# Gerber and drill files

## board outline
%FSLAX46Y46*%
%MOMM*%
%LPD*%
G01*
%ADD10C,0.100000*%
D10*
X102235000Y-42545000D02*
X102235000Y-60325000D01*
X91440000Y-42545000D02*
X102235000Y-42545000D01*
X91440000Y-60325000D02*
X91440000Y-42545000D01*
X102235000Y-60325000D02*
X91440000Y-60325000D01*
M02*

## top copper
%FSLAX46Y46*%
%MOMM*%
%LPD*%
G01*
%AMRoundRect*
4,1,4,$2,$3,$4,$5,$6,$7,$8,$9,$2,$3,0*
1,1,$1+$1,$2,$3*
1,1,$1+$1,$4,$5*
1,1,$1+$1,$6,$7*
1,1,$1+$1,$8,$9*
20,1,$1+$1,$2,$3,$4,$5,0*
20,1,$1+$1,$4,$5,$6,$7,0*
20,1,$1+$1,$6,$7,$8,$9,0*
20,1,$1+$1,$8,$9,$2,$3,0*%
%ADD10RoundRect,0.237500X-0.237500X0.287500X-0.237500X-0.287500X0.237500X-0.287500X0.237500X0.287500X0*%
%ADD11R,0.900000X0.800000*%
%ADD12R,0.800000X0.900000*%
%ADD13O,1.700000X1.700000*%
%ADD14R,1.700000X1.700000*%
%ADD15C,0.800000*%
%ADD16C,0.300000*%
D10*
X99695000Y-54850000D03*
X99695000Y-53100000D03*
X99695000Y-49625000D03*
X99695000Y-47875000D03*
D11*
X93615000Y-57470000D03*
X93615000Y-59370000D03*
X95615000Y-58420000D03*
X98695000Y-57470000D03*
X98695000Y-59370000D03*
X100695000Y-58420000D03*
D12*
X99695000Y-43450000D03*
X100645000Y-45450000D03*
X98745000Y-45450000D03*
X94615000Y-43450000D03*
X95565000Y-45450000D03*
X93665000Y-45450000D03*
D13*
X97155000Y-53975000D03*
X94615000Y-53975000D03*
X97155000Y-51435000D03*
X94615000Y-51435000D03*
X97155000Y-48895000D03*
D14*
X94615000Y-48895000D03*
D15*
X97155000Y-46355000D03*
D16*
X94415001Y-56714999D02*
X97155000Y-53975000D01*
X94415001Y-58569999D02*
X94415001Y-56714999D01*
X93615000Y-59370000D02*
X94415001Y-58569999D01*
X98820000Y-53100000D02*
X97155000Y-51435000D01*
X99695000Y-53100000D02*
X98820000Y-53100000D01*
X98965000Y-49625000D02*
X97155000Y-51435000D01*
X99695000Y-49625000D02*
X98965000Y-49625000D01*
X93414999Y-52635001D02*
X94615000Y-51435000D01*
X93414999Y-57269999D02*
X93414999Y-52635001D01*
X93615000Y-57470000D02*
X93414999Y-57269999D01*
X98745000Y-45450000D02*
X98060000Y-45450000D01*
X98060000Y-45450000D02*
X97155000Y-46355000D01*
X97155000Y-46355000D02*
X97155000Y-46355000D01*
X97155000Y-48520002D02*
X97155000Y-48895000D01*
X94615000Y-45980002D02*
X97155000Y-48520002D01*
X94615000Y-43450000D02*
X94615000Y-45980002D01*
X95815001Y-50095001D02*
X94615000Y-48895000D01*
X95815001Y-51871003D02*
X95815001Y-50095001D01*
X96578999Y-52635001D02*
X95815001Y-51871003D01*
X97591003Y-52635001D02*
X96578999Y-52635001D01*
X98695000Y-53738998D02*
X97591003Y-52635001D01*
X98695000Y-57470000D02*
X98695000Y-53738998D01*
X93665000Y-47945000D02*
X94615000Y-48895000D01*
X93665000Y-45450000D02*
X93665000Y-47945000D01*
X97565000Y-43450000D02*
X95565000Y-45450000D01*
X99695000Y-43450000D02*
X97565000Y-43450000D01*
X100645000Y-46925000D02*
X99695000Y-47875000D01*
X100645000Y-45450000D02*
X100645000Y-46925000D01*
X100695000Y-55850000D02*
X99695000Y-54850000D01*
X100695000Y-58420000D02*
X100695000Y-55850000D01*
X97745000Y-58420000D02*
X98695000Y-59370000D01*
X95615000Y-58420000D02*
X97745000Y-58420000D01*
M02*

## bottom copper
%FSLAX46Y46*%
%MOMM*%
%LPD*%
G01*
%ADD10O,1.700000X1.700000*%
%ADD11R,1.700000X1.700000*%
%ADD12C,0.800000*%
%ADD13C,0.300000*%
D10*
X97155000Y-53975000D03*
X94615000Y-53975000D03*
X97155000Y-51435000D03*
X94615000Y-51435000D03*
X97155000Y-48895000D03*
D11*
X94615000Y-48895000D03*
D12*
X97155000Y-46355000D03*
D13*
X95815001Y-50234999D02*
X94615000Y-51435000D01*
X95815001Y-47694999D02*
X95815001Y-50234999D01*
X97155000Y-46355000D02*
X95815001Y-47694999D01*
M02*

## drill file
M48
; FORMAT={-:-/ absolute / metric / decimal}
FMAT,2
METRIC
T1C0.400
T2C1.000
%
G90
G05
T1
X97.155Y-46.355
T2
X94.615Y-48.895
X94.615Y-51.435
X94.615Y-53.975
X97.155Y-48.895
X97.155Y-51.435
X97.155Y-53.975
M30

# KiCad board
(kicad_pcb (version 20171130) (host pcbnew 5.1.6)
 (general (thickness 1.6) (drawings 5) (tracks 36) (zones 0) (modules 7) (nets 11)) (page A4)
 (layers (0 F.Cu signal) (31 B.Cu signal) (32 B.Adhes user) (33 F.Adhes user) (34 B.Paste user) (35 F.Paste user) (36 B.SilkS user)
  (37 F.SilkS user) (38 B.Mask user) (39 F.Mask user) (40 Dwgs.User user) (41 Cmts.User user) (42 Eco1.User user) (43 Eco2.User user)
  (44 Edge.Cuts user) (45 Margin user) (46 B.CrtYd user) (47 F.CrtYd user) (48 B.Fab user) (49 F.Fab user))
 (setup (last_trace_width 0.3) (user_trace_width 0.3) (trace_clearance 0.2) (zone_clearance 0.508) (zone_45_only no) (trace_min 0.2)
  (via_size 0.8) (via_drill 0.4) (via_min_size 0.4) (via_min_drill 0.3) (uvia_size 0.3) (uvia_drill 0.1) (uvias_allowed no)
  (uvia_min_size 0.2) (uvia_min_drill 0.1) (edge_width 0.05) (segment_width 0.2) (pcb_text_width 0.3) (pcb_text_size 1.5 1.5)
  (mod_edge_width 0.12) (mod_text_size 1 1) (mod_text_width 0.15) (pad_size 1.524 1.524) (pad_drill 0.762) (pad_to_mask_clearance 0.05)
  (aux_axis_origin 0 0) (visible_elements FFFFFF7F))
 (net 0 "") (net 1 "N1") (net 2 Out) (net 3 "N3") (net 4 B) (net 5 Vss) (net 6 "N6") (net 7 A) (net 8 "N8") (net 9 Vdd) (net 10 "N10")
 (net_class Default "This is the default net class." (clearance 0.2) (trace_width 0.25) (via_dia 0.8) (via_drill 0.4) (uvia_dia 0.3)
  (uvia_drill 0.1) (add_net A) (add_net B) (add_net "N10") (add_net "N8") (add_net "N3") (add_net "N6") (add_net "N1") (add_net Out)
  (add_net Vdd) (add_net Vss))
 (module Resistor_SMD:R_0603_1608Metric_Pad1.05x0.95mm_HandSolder (layer F.Cu) (at 99.695 53.975 270)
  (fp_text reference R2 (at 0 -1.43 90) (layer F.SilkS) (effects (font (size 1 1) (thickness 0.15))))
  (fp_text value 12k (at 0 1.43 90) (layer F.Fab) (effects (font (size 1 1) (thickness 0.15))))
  (pad 2 smd roundrect (at 0.875 0 270) (size 1.05 0.95) (layers F.Cu F.Paste F.Mask) (roundrect_rratio 0.25) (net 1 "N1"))
  (pad 1 smd roundrect (at -0.875 0 270) (size 1.05 0.95) (layers F.Cu F.Paste F.Mask) (roundrect_rratio 0.25) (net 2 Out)))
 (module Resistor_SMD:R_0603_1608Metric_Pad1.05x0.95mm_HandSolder (layer F.Cu) (at 99.695 48.75 270)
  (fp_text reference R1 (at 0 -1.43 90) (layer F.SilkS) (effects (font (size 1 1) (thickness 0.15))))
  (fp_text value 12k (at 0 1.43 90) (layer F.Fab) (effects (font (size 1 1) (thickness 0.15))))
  (pad 2 smd roundrect (at 0.875 0 270) (size 1.05 0.95) (layers F.Cu F.Paste F.Mask) (roundrect_rratio 0.25) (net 2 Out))
  (pad 1 smd roundrect (at -0.875 0 270) (size 1.05 0.95) (layers F.Cu F.Paste F.Mask) (roundrect_rratio 0.25) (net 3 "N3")))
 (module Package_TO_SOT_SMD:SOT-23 (layer F.Cu) (at 94.615 58.42)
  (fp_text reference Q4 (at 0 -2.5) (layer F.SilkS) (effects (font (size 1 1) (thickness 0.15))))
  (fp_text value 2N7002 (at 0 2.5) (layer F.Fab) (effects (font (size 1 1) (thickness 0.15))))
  (pad 1 smd rect (at -1 -0.95) (size 0.9 0.8) (layers F.Cu F.Paste F.Mask) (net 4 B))
  (pad 2 smd rect (at -1 0.95) (size 0.9 0.8) (layers F.Cu F.Paste F.Mask) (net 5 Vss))
  (pad 3 smd rect (at 1 0) (size 0.9 0.8) (layers F.Cu F.Paste F.Mask) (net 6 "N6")))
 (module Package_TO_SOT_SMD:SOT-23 (layer F.Cu) (at 99.695 58.42)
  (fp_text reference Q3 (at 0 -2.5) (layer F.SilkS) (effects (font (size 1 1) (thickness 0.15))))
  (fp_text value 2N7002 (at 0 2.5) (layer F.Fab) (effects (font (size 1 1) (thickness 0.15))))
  (pad 1 smd rect (at -1 -0.95) (size 0.9 0.8) (layers F.Cu F.Paste F.Mask) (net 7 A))
  (pad 2 smd rect (at -1 0.95) (size 0.9 0.8) (layers F.Cu F.Paste F.Mask) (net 6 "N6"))
  (pad 3 smd rect (at 1 0) (size 0.9 0.8) (layers F.Cu F.Paste F.Mask) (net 1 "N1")))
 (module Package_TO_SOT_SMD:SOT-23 (layer F.Cu) (at 99.695 44.45 90)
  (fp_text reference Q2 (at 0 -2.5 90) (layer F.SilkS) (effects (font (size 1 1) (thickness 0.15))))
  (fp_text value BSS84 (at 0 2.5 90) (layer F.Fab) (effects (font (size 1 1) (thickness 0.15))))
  (pad 3 smd rect (at 1 0 90) (size 0.9 0.8) (layers F.Cu F.Paste F.Mask) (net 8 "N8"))
  (pad 2 smd rect (at -1 0.95 90) (size 0.9 0.8) (layers F.Cu F.Paste F.Mask) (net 3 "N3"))
  (pad 1 smd rect (at -1 -0.95 90) (size 0.9 0.8) (layers F.Cu F.Paste F.Mask) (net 4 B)))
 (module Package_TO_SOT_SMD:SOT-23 (layer F.Cu) (at 94.615 44.45 90)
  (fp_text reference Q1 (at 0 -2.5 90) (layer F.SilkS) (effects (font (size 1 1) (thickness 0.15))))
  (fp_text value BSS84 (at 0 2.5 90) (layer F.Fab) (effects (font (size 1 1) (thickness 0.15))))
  (pad 3 smd rect (at 1 0 90) (size 0.9 0.8) (layers F.Cu F.Paste F.Mask) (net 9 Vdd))
  (pad 2 smd rect (at -1 0.95 90) (size 0.9 0.8) (layers F.Cu F.Paste F.Mask) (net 8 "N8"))
  (pad 1 smd rect (at -1 -0.95 90) (size 0.9 0.8) (layers F.Cu F.Paste F.Mask) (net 7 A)))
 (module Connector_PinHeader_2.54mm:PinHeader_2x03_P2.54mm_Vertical (layer F.Cu) (at 94.615 48.895)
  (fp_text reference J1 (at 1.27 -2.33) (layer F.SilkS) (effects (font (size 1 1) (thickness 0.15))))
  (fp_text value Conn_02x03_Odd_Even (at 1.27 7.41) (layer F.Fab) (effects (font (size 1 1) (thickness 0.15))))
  (pad 6 thru_hole oval (at 2.54 5.08) (size 1.7 1.7) (drill 1) (layers *.Cu *.Mask) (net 5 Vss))
  (pad 5 thru_hole oval (at 0 5.08) (size 1.7 1.7) (drill 1) (layers *.Cu *.Mask) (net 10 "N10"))
  (pad 4 thru_hole oval (at 2.54 2.54) (size 1.7 1.7) (drill 1) (layers *.Cu *.Mask) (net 2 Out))
  (pad 3 thru_hole oval (at 0 2.54) (size 1.7 1.7) (drill 1) (layers *.Cu *.Mask) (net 4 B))
  (pad 2 thru_hole oval (at 2.54 0) (size 1.7 1.7) (drill 1) (layers *.Cu *.Mask) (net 9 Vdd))
  (pad 1 thru_hole rect (at 0 0) (size 1.7 1.7) (drill 1) (layers *.Cu *.Mask) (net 7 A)))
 (gr_line (start 102.235 42.545) (end 102.235 60.325) (layer Edge.Cuts) (width 0.1))
 (gr_line (start 91.44 42.545) (end 102.235 42.545) (layer Edge.Cuts) (width 0.1))
 (gr_line (start 91.44 60.325) (end 91.44 42.545) (layer Edge.Cuts) (width 0.1))
 (gr_line (start 102.235 60.325) (end 91.44 60.325) (layer Edge.Cuts) (width 0.1))
 (segment (start 94.415001 56.714999) (end 97.155 53.975) (width 0.3) (layer F.Cu) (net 5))
 (segment (start 94.415001 58.569999) (end 94.415001 56.714999) (width 0.3) (layer F.Cu) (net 5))
 (segment (start 93.615 59.37) (end 94.415001 58.569999) (width 0.3) (layer F.Cu) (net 5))
 (segment (start 98.82 53.1) (end 97.155 51.435) (width 0.3) (layer F.Cu) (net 2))
 (segment (start 99.695 53.1) (end 98.82 53.1) (width 0.3) (layer F.Cu) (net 2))
 (segment (start 98.965 49.625) (end 97.155 51.435) (width 0.3) (layer F.Cu) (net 2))
 (segment (start 99.695 49.625) (end 98.965 49.625) (width 0.3) (layer F.Cu) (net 2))
 (segment (start 93.414999 52.635001) (end 94.615 51.435) (width 0.3) (layer F.Cu) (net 4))
 (segment (start 93.414999 57.269999) (end 93.414999 52.635001) (width 0.3) (layer F.Cu) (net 4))
 (segment (start 93.615 57.47) (end 93.414999 57.269999) (width 0.3) (layer F.Cu) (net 4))
 (segment (start 98.745 45.45) (end 98.06 45.45) (width 0.3) (layer F.Cu) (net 4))
 (segment (start 98.06 45.45) (end 97.155 46.355) (width 0.3) (layer F.Cu) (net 4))
 (segment (start 97.155 46.355) (end 97.155 46.355) (width 0.3) (layer F.Cu) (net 4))
 (via (at 97.155 46.355) (size 0.8) (drill 0.4) (layers F.Cu B.Cu) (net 4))
 (segment (start 95.815001 50.234999) (end 94.615 51.435) (width 0.3) (layer B.Cu) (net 4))
 (segment (start 95.815001 47.694999) (end 95.815001 50.234999) (width 0.3) (layer B.Cu) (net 4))
 (segment (start 97.155 46.355) (end 95.815001 47.694999) (width 0.3) (layer B.Cu) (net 4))
 (segment (start 97.155 48.520002) (end 97.155 48.895) (width 0.3) (layer F.Cu) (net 9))
 (segment (start 94.615 45.980002) (end 97.155 48.520002) (width 0.3) (layer F.Cu) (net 9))
 (segment (start 94.615 43.45) (end 94.615 45.980002) (width 0.3) (layer F.Cu) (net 9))
 (segment (start 95.815001 50.095001) (end 94.615 48.895) (width 0.3) (layer F.Cu) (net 7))
 (segment (start 95.815001 51.871003) (end 95.815001 50.095001) (width 0.3) (layer F.Cu) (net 7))
 (segment (start 96.578999 52.635001) (end 95.815001 51.871003) (width 0.3) (layer F.Cu) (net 7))
 (segment (start 97.591003 52.635001) (end 96.578999 52.635001) (width 0.3) (layer F.Cu) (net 7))
 (segment (start 98.695 53.738998) (end 97.591003 52.635001) (width 0.3) (layer F.Cu) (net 7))
 (segment (start 98.695 57.47) (end 98.695 53.738998) (width 0.3) (layer F.Cu) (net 7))
 (segment (start 93.665 47.945) (end 94.615 48.895) (width 0.3) (layer F.Cu) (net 7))
 (segment (start 93.665 45.45) (end 93.665 47.945) (width 0.3) (layer F.Cu) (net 7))
 (segment (start 97.565 43.45) (end 95.565 45.45) (width 0.3) (layer F.Cu) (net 8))
 (segment (start 99.695 43.45) (end 97.565 43.45) (width 0.3) (layer F.Cu) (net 8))
 (segment (start 100.645 46.925) (end 99.695 47.875) (width 0.3) (layer F.Cu) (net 3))
 (segment (start 100.645 45.45) (end 100.645 46.925) (width 0.3) (layer F.Cu) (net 3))
 (segment (start 100.695 55.85) (end 99.695 54.85) (width 0.3) (layer F.Cu) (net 1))
 (segment (start 100.695 58.42) (end 100.695 55.85) (width 0.3) (layer F.Cu) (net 1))
 (segment (start 97.745 58.42) (end 98.695 59.37) (width 0.3) (layer F.Cu) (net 6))
 (segment (start 95.615 58.42) (end 97.745 58.42) (width 0.3) (layer F.Cu) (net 6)))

